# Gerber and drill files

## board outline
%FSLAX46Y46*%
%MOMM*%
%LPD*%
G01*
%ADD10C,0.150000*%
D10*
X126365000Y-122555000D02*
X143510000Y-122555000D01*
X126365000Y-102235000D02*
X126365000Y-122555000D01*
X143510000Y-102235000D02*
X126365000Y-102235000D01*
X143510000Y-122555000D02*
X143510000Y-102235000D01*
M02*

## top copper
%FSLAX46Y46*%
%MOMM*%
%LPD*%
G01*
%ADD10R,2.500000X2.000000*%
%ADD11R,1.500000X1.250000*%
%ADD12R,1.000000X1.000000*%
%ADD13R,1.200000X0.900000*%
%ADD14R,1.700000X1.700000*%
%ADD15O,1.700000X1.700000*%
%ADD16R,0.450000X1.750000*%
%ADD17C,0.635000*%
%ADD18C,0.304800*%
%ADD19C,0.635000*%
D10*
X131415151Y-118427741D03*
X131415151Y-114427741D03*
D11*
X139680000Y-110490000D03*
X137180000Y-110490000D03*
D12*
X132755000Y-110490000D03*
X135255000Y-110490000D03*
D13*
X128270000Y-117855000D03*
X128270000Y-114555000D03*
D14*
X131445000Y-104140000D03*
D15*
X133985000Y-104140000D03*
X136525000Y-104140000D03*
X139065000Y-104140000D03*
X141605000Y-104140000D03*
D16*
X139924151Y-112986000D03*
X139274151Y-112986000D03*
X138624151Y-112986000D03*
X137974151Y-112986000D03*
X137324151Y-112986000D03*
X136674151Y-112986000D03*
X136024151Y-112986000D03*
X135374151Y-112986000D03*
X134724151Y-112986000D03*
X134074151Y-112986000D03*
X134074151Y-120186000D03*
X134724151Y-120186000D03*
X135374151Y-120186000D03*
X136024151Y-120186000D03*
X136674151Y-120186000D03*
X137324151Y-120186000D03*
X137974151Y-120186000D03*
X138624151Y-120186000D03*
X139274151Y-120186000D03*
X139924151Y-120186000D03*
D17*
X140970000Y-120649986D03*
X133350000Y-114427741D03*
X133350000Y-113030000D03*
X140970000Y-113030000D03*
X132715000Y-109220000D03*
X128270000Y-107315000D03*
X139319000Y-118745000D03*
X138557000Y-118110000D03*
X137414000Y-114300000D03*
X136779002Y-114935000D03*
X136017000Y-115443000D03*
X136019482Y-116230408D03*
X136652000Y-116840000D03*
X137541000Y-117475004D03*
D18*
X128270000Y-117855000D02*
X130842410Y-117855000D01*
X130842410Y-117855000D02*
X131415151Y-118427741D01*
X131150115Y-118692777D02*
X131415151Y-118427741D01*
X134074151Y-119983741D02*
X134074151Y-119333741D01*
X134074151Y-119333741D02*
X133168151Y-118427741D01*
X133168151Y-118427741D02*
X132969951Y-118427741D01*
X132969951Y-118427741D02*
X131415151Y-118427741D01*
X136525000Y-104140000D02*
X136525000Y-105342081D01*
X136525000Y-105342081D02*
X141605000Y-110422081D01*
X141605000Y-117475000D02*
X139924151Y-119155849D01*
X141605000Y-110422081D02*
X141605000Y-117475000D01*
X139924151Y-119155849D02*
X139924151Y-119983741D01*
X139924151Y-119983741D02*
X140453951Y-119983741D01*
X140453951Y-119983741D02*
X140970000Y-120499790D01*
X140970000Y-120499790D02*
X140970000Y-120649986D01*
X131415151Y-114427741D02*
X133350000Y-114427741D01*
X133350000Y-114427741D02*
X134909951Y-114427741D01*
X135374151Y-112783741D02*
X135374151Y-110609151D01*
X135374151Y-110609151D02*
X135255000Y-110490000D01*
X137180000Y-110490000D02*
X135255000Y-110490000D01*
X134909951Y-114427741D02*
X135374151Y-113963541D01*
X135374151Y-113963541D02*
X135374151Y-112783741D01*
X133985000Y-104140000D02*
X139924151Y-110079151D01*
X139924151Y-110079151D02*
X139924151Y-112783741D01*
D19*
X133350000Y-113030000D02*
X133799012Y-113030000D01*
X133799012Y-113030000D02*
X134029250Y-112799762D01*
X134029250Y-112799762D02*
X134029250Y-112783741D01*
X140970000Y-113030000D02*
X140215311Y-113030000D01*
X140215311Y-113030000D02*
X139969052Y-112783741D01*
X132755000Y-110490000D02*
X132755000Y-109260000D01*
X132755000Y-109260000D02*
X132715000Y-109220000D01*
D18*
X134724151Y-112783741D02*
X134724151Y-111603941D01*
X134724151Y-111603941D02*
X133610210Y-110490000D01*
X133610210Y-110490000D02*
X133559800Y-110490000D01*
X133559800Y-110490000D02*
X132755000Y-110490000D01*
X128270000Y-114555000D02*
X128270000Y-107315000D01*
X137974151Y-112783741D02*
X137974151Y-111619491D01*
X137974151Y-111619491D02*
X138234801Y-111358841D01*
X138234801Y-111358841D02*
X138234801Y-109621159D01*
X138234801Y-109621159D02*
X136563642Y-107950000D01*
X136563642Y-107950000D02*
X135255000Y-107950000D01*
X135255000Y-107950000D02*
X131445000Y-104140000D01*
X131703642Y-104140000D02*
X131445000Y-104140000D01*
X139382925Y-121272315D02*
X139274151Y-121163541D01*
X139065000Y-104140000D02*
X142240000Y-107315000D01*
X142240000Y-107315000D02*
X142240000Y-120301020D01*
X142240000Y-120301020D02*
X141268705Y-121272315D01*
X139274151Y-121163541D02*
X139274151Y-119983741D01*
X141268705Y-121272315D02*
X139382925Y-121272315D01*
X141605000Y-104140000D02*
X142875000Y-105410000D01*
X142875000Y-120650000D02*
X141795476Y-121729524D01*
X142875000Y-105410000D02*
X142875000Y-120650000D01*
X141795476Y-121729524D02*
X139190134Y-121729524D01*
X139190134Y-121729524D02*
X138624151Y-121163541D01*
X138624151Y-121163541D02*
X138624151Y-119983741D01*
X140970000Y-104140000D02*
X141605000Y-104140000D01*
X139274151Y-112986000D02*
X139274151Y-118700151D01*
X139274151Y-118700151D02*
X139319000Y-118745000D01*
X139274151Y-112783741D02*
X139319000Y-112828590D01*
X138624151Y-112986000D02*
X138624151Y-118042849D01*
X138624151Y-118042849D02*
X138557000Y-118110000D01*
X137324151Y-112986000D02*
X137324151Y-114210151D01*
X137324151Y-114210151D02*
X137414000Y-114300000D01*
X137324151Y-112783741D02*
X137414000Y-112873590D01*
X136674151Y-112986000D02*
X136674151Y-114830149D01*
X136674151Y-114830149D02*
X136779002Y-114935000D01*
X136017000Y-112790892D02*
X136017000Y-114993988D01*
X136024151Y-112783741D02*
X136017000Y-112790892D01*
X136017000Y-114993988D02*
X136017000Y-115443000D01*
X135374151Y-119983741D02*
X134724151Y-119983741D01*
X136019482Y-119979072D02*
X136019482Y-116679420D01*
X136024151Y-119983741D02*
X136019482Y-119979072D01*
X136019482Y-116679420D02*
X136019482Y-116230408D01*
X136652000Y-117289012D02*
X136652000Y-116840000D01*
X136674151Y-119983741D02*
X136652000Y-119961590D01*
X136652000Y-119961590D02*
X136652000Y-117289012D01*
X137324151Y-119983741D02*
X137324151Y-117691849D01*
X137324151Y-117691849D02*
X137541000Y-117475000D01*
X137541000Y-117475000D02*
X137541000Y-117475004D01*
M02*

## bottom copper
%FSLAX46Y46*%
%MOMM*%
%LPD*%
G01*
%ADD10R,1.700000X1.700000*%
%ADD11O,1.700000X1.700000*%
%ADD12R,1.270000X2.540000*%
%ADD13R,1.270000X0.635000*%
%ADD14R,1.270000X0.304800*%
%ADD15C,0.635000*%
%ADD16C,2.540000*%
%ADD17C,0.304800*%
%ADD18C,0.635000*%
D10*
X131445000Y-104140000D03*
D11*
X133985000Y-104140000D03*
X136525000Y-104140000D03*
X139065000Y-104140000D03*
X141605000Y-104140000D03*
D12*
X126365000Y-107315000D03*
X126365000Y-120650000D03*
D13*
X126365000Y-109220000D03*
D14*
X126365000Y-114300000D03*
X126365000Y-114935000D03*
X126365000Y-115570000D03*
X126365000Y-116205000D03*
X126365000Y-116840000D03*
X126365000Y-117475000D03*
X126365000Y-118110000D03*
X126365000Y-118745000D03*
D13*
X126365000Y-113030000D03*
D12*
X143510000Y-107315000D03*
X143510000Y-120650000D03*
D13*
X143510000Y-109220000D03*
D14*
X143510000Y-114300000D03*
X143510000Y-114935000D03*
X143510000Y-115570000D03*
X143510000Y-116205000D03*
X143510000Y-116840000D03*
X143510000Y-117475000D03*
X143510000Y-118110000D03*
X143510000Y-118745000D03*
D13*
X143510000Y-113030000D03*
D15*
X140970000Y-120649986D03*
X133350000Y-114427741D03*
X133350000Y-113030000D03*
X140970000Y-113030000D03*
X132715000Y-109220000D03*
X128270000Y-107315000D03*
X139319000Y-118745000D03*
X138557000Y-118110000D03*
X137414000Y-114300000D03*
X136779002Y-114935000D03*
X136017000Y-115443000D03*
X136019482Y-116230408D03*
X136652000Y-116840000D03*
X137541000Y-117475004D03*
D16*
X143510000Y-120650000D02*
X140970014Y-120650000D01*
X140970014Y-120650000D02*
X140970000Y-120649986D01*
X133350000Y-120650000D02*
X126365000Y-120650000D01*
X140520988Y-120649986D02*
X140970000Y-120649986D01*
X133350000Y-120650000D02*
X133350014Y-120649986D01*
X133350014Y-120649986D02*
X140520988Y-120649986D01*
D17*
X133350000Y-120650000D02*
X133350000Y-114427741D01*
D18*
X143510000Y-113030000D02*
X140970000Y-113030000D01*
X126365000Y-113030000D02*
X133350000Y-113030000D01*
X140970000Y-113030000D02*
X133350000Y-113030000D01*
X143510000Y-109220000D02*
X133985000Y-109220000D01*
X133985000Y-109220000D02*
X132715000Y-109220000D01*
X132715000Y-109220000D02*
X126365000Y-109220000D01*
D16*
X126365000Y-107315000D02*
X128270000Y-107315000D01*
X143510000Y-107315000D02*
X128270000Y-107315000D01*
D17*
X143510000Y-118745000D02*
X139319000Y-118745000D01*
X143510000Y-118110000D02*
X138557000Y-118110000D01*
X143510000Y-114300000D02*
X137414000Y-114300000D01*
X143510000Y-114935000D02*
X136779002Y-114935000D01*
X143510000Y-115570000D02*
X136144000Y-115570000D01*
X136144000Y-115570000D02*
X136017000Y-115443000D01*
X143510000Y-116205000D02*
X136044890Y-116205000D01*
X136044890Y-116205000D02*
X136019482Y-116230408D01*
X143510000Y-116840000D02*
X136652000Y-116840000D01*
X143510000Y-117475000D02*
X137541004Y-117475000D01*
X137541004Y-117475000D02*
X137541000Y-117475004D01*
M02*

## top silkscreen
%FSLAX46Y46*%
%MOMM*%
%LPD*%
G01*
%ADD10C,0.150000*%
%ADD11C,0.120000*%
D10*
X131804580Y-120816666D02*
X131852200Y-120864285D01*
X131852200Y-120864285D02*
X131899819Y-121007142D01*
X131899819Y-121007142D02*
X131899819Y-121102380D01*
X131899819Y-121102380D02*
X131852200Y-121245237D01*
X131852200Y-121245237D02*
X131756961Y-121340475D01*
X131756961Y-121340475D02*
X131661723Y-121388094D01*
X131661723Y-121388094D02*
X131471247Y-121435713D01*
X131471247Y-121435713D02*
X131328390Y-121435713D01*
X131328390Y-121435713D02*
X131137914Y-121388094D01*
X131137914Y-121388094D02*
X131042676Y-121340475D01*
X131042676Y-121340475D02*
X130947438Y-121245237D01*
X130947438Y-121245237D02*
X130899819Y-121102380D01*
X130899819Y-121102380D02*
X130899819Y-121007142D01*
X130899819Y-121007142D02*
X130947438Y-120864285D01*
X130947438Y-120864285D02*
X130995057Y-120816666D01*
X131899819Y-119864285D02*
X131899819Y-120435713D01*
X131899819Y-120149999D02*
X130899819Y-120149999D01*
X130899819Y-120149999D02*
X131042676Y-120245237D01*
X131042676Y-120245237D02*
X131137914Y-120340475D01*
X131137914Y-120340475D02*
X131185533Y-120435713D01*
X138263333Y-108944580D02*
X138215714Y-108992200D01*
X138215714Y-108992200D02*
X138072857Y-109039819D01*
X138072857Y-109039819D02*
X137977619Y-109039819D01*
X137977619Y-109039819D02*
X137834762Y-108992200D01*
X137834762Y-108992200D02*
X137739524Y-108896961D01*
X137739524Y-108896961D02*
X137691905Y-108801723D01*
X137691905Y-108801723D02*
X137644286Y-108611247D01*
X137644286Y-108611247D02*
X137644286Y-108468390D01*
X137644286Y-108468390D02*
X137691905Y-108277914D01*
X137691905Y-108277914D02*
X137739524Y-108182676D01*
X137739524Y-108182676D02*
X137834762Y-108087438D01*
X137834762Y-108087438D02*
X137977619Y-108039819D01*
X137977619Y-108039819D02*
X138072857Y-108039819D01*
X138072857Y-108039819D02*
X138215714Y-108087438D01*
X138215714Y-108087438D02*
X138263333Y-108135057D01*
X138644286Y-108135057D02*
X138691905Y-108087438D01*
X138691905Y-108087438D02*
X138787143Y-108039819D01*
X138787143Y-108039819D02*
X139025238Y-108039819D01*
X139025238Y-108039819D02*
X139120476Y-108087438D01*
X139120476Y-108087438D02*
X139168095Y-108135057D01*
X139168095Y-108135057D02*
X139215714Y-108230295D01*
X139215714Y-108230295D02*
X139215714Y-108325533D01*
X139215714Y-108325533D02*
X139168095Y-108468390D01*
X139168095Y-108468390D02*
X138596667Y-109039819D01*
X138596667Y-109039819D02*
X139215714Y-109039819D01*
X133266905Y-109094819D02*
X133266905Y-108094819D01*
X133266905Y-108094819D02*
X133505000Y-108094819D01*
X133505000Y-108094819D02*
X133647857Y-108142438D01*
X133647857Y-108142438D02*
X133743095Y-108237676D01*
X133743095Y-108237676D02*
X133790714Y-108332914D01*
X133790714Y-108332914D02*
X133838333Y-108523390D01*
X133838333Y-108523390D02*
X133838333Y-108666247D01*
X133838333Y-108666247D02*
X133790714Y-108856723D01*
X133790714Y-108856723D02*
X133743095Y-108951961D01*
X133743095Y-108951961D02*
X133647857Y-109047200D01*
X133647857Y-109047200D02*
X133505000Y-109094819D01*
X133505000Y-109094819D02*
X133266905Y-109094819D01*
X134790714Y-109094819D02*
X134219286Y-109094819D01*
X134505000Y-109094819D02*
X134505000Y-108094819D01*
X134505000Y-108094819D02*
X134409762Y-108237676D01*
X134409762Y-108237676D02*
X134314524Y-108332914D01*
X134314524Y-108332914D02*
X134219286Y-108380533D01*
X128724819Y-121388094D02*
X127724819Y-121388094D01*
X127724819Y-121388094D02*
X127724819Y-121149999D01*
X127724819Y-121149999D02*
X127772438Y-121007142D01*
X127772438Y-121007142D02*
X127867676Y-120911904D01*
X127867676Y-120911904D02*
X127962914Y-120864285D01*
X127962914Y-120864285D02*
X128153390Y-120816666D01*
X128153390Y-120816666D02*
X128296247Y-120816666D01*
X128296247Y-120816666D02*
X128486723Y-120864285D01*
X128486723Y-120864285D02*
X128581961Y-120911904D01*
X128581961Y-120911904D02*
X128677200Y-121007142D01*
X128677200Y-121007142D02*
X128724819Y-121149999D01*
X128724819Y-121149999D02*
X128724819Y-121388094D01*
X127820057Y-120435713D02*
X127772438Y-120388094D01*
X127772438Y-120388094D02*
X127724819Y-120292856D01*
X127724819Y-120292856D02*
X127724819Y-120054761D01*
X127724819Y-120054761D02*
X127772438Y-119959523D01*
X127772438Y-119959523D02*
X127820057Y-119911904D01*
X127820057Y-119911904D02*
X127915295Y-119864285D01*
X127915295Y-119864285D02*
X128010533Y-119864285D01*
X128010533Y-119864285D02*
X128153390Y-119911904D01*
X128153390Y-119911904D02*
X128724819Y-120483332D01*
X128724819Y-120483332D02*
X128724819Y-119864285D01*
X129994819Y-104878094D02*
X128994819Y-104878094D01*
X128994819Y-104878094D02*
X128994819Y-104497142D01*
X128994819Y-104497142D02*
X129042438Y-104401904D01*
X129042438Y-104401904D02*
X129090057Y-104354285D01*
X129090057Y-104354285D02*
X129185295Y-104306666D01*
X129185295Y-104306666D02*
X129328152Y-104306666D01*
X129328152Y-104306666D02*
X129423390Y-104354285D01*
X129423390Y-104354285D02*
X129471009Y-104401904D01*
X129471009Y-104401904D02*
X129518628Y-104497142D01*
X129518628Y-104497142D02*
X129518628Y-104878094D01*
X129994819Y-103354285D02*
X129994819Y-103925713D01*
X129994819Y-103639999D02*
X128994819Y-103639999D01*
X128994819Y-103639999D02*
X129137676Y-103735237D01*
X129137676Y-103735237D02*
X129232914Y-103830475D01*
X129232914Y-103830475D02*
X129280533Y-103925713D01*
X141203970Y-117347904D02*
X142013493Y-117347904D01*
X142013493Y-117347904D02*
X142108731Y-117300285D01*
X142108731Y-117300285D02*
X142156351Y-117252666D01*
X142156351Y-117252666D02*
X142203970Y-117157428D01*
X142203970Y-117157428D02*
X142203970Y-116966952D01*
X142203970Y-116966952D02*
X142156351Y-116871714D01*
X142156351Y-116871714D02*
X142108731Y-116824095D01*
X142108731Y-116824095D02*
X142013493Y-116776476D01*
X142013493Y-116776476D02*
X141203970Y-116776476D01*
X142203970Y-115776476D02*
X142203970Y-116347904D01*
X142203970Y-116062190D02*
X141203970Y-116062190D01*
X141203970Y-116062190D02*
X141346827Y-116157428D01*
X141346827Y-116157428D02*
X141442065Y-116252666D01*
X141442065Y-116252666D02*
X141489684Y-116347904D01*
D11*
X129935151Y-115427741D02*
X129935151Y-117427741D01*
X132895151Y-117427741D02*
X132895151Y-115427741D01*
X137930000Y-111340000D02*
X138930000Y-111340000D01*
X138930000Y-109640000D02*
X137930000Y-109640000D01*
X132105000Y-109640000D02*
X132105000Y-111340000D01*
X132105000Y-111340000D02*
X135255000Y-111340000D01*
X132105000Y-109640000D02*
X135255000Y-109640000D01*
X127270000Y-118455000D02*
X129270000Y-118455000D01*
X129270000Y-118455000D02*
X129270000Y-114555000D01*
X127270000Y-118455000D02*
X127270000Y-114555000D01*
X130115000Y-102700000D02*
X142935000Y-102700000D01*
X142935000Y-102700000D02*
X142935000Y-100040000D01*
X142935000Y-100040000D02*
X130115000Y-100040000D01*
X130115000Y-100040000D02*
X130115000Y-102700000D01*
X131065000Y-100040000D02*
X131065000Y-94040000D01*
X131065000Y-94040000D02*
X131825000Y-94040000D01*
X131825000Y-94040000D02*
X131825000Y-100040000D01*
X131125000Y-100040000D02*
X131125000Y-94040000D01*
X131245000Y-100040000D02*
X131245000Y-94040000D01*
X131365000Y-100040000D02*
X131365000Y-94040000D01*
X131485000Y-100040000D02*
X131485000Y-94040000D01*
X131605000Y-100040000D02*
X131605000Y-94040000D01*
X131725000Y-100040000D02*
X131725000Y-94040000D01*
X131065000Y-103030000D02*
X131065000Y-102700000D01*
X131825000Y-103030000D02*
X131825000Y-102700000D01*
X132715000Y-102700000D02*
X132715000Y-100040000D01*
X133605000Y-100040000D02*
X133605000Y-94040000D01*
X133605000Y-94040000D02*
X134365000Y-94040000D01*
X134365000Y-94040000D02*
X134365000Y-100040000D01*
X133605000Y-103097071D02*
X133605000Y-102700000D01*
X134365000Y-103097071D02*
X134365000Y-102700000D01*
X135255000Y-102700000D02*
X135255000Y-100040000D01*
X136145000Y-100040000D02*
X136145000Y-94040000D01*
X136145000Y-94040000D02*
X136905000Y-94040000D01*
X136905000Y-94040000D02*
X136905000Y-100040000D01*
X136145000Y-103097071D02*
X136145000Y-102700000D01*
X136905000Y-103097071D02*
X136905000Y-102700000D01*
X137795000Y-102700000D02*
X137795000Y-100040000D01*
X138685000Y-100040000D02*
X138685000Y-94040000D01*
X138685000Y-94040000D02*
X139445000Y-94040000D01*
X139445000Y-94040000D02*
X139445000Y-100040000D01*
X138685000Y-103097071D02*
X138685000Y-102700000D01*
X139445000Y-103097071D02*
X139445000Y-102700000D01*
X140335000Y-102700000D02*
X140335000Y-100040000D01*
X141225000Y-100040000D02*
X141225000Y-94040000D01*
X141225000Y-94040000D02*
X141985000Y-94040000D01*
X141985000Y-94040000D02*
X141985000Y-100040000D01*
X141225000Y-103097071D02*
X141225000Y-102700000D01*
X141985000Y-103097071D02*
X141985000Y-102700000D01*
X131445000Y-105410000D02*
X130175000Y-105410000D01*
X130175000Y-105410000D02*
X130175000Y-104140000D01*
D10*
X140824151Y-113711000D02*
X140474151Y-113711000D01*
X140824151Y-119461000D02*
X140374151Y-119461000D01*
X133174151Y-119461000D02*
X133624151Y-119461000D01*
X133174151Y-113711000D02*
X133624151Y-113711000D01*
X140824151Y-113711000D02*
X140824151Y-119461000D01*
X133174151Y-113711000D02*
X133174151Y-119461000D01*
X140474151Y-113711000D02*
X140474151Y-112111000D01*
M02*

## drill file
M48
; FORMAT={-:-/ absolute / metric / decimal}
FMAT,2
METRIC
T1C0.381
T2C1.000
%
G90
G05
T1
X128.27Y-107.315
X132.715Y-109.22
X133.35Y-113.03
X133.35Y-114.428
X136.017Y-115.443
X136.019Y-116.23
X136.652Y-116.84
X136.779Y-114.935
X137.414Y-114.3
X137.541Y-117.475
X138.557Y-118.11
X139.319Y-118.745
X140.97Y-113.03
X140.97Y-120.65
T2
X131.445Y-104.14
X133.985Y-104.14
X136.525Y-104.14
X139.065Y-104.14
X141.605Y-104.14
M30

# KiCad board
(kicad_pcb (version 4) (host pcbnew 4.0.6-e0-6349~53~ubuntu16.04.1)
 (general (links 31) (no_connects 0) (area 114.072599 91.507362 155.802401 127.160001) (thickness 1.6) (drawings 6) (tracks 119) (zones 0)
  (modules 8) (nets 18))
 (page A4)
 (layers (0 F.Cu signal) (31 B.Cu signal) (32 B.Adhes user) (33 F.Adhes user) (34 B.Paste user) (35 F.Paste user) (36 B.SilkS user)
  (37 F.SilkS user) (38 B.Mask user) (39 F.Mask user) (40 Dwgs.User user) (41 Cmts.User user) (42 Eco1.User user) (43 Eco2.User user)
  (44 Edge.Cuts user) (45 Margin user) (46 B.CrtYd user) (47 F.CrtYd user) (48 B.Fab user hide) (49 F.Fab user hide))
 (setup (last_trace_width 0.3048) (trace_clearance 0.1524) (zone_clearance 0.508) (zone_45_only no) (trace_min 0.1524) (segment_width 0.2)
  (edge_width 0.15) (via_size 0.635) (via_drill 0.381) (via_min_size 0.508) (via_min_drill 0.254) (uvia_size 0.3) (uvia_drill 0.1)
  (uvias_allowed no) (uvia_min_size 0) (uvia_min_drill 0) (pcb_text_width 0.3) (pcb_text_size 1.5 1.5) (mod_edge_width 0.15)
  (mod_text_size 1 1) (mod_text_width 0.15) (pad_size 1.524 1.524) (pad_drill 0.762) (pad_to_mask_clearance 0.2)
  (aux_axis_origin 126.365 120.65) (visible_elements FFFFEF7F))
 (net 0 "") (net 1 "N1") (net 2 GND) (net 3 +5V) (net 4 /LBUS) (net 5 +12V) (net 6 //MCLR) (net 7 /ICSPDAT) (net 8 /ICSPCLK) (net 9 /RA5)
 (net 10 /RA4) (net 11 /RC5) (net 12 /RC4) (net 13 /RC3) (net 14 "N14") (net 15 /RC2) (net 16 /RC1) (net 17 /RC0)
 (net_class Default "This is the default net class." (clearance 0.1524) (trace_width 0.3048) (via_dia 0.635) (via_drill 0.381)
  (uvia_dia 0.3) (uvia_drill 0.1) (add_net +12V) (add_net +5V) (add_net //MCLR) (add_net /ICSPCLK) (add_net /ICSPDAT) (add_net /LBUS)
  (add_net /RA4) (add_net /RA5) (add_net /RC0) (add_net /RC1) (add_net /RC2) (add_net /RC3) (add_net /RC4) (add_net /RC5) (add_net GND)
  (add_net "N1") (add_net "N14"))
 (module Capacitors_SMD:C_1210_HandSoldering (layer F.Cu) (at 131.415151 116.427741 90)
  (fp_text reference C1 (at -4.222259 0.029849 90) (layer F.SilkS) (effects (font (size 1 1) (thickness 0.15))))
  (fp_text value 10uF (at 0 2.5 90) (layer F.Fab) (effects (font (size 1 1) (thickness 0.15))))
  (fp_line (start 1 -1.48) (end -1 -1.48) (layer F.SilkS) (width 0.12))
  (fp_line (start -1 1.48) (end 1 1.48) (layer F.SilkS) (width 0.12))
  (pad 1 smd rect (at -2 0 90) (size 2 2.5) (layers F.Cu F.Paste F.Mask) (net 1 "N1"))
  (pad 2 smd rect (at 2 0 90) (size 2 2.5) (layers F.Cu F.Paste F.Mask) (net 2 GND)))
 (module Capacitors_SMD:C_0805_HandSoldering (layer F.Cu) (at 138.43 110.49 180)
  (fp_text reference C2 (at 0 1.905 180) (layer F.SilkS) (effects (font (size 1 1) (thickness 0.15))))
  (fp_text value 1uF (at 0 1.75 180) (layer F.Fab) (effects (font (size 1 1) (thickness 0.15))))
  (fp_line (start 0.5 -0.85) (end -0.5 -0.85) (layer F.SilkS) (width 0.12))
  (fp_line (start -0.5 0.85) (end 0.5 0.85) (layer F.SilkS) (width 0.12))
  (pad 1 smd rect (at -1.25 0 180) (size 1.5 1.25) (layers F.Cu F.Paste F.Mask) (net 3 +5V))
  (pad 2 smd rect (at 1.25 0 180) (size 1.5 1.25) (layers F.Cu F.Paste F.Mask) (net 2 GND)))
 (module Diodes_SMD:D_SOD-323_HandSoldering (layer F.Cu) (at 134.005 110.49)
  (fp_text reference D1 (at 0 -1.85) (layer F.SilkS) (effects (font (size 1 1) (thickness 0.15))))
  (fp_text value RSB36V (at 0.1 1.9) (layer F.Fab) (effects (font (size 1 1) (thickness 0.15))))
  (fp_line (start -1.9 -0.85) (end -1.9 0.85) (layer F.SilkS) (width 0.12))
  (fp_line (start -1.9 0.85) (end 1.25 0.85) (layer F.SilkS) (width 0.12))
  (fp_line (start -1.9 -0.85) (end 1.25 -0.85) (layer F.SilkS) (width 0.12))
  (pad 1 smd rect (at -1.25 0) (size 1 1) (layers F.Cu F.Paste F.Mask) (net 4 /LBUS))
  (pad 2 smd rect (at 1.25 0) (size 1 1) (layers F.Cu F.Paste F.Mask) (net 2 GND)))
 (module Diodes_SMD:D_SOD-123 (layer F.Cu) (at 128.27 116.205 90)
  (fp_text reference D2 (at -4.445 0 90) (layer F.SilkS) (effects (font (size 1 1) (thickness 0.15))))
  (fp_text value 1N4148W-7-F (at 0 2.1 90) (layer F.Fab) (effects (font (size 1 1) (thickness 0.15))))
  (fp_line (start -2.25 -1) (end -2.25 1) (layer F.SilkS) (width 0.12))
  (fp_line (start -2.25 1) (end 1.65 1) (layer F.SilkS) (width 0.12))
  (fp_line (start -2.25 -1) (end 1.65 -1) (layer F.SilkS) (width 0.12))
  (pad 1 smd rect (at -1.65 0 90) (size 0.9 1.2) (layers F.Cu F.Paste F.Mask) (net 1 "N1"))
  (pad 2 smd rect (at 1.65 0 90) (size 0.9 1.2) (layers F.Cu F.Paste F.Mask) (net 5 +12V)))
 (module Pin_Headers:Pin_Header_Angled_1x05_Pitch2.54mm (layer F.Cu) (at 131.445 104.14 90)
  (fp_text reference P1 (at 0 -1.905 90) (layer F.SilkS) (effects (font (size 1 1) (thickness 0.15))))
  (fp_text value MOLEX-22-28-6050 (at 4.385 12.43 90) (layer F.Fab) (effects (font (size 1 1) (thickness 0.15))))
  (fp_line (start 1.44 -1.33) (end 1.44 11.49) (layer F.SilkS) (width 0.12))
  (fp_line (start 1.44 11.49) (end 4.1 11.49) (layer F.SilkS) (width 0.12))
  (fp_line (start 4.1 11.49) (end 4.1 -1.33) (layer F.SilkS) (width 0.12))
  (fp_line (start 4.1 -1.33) (end 1.44 -1.33) (layer F.SilkS) (width 0.12))
  (fp_line (start 4.1 -0.38) (end 10.1 -0.38) (layer F.SilkS) (width 0.12))
  (fp_line (start 10.1 -0.38) (end 10.1 0.38) (layer F.SilkS) (width 0.12))
  (fp_line (start 10.1 0.38) (end 4.1 0.38) (layer F.SilkS) (width 0.12))
  (fp_line (start 4.1 -0.32) (end 10.1 -0.32) (layer F.SilkS) (width 0.12))
  (fp_line (start 4.1 -0.2) (end 10.1 -0.2) (layer F.SilkS) (width 0.12))
  (fp_line (start 4.1 -0.08) (end 10.1 -0.08) (layer F.SilkS) (width 0.12))
  (fp_line (start 4.1 0.04) (end 10.1 0.04) (layer F.SilkS) (width 0.12))
  (fp_line (start 4.1 0.16) (end 10.1 0.16) (layer F.SilkS) (width 0.12))
  (fp_line (start 4.1 0.28) (end 10.1 0.28) (layer F.SilkS) (width 0.12))
  (fp_line (start 1.11 -0.38) (end 1.44 -0.38) (layer F.SilkS) (width 0.12))
  (fp_line (start 1.11 0.38) (end 1.44 0.38) (layer F.SilkS) (width 0.12))
  (fp_line (start 1.44 1.27) (end 4.1 1.27) (layer F.SilkS) (width 0.12))
  (fp_line (start 4.1 2.16) (end 10.1 2.16) (layer F.SilkS) (width 0.12))
  (fp_line (start 10.1 2.16) (end 10.1 2.92) (layer F.SilkS) (width 0.12))
  (fp_line (start 10.1 2.92) (end 4.1 2.92) (layer F.SilkS) (width 0.12))
  (fp_line (start 1.042929 2.16) (end 1.44 2.16) (layer F.SilkS) (width 0.12))
  (fp_line (start 1.042929 2.92) (end 1.44 2.92) (layer F.SilkS) (width 0.12))
  (fp_line (start 1.44 3.81) (end 4.1 3.81) (layer F.SilkS) (width 0.12))
  (fp_line (start 4.1 4.7) (end 10.1 4.7) (layer F.SilkS) (width 0.12))
  (fp_line (start 10.1 4.7) (end 10.1 5.46) (layer F.SilkS) (width 0.12))
  (fp_line (start 10.1 5.46) (end 4.1 5.46) (layer F.SilkS) (width 0.12))
  (fp_line (start 1.042929 4.7) (end 1.44 4.7) (layer F.SilkS) (width 0.12))
  (fp_line (start 1.042929 5.46) (end 1.44 5.46) (layer F.SilkS) (width 0.12))
  (fp_line (start 1.44 6.35) (end 4.1 6.35) (layer F.SilkS) (width 0.12))
  (fp_line (start 4.1 7.24) (end 10.1 7.24) (layer F.SilkS) (width 0.12))
  (fp_line (start 10.1 7.24) (end 10.1 8) (layer F.SilkS) (width 0.12))
  (fp_line (start 10.1 8) (end 4.1 8) (layer F.SilkS) (width 0.12))
  (fp_line (start 1.042929 7.24) (end 1.44 7.24) (layer F.SilkS) (width 0.12))
  (fp_line (start 1.042929 8) (end 1.44 8) (layer F.SilkS) (width 0.12))
  (fp_line (start 1.44 8.89) (end 4.1 8.89) (layer F.SilkS) (width 0.12))
  (fp_line (start 4.1 9.78) (end 10.1 9.78) (layer F.SilkS) (width 0.12))
  (fp_line (start 10.1 9.78) (end 10.1 10.54) (layer F.SilkS) (width 0.12))
  (fp_line (start 10.1 10.54) (end 4.1 10.54) (layer F.SilkS) (width 0.12))
  (fp_line (start 1.042929 9.78) (end 1.44 9.78) (layer F.SilkS) (width 0.12))
  (fp_line (start 1.042929 10.54) (end 1.44 10.54) (layer F.SilkS) (width 0.12))
  (fp_line (start -1.27 0) (end -1.27 -1.27) (layer F.SilkS) (width 0.12))
  (fp_line (start -1.27 -1.27) (end 0 -1.27) (layer F.SilkS) (width 0.12))
  (pad 1 thru_hole rect (at 0 0 90) (size 1.7 1.7) (drill 1) (layers *.Cu *.Mask) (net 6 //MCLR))
  (pad 2 thru_hole oval (at 0 2.54 90) (size 1.7 1.7) (drill 1) (layers *.Cu *.Mask) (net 3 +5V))
  (pad 3 thru_hole oval (at 0 5.08 90) (size 1.7 1.7) (drill 1) (layers *.Cu *.Mask) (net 2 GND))
  (pad 4 thru_hole oval (at 0 7.62 90) (size 1.7 1.7) (drill 1) (layers *.Cu *.Mask) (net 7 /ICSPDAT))
  (pad 5 thru_hole oval (at 0 10.16 90) (size 1.7 1.7) (drill 1) (layers *.Cu *.Mask) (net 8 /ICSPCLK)))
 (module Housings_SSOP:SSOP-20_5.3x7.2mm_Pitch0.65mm (layer F.Cu) (at 136.999151 116.586 270)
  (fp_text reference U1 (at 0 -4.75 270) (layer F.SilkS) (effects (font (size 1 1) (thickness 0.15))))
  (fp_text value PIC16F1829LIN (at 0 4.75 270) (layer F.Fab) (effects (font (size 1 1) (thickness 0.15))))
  (fp_line (start -2.875 -3.825) (end -2.875 -3.475) (layer F.SilkS) (width 0.15))
  (fp_line (start 2.875 -3.825) (end 2.875 -3.375) (layer F.SilkS) (width 0.15))
  (fp_line (start 2.875 3.825) (end 2.875 3.375) (layer F.SilkS) (width 0.15))
  (fp_line (start -2.875 3.825) (end -2.875 3.375) (layer F.SilkS) (width 0.15))
  (fp_line (start -2.875 -3.825) (end 2.875 -3.825) (layer F.SilkS) (width 0.15))
  (fp_line (start -2.875 3.825) (end 2.875 3.825) (layer F.SilkS) (width 0.15))
  (fp_line (start -2.875 -3.475) (end -4.475 -3.475) (layer F.SilkS) (width 0.15))
  (pad 1 smd rect (at -3.6 -2.925 270) (size 1.75 0.45) (layers F.Cu F.Paste F.Mask) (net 3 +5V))
  (pad 2 smd rect (at -3.6 -2.275 270) (size 1.75 0.45) (layers F.Cu F.Paste F.Mask) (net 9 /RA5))
  (pad 3 smd rect (at -3.6 -1.625 270) (size 1.75 0.45) (layers F.Cu F.Paste F.Mask) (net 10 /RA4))
  (pad 4 smd rect (at -3.6 -0.975 270) (size 1.75 0.45) (layers F.Cu F.Paste F.Mask) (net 6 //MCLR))
  (pad 5 smd rect (at -3.6 -0.325 270) (size 1.75 0.45) (layers F.Cu F.Paste F.Mask) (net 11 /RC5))
  (pad 6 smd rect (at -3.6 0.325 270) (size 1.75 0.45) (layers F.Cu F.Paste F.Mask) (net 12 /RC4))
  (pad 7 smd rect (at -3.6 0.975 270) (size 1.75 0.45) (layers F.Cu F.Paste F.Mask) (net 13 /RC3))
  (pad 8 smd rect (at -3.6 1.625 270) (size 1.75 0.45) (layers F.Cu F.Paste F.Mask) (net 2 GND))
  (pad 9 smd rect (at -3.6 2.275 270) (size 1.75 0.45) (layers F.Cu F.Paste F.Mask) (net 4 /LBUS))
  (pad 10 smd rect (at -3.6 2.925 270) (size 1.75 0.45) (layers F.Cu F.Paste F.Mask) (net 3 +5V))
  (pad 11 smd rect (at 3.6 2.925 270) (size 1.75 0.45) (layers F.Cu F.Paste F.Mask) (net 1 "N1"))
  (pad 12 smd rect (at 3.6 2.275 270) (size 1.75 0.45) (layers F.Cu F.Paste F.Mask) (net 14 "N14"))
  (pad 13 smd rect (at 3.6 1.625 270) (size 1.75 0.45) (layers F.Cu F.Paste F.Mask) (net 14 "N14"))
  (pad 14 smd rect (at 3.6 0.975 270) (size 1.75 0.45) (layers F.Cu F.Paste F.Mask) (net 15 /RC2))
  (pad 15 smd rect (at 3.6 0.325 270) (size 1.75 0.45) (layers F.Cu F.Paste F.Mask) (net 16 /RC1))
  (pad 16 smd rect (at 3.6 -0.325 270) (size 1.75 0.45) (layers F.Cu F.Paste F.Mask) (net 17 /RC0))
  (pad 17 smd rect (at 3.6 -0.975 270) (size 1.75 0.45) (layers F.Cu F.Paste F.Mask))
  (pad 18 smd rect (at 3.6 -1.625 270) (size 1.75 0.45) (layers F.Cu F.Paste F.Mask) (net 8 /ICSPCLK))
  (pad 19 smd rect (at 3.6 -2.275 270) (size 1.75 0.45) (layers F.Cu F.Paste F.Mask) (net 7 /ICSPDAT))
  (pad 20 smd rect (at 3.6 -2.925 270) (size 1.75 0.45) (layers F.Cu F.Paste F.Mask) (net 2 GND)))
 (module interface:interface (layer F.Cu) (at 126.365 102.87)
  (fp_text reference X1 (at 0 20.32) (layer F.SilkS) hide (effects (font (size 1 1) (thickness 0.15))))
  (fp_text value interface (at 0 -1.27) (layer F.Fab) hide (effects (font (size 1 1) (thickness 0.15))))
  (pad 1 smd rect (at 0 4.445) (size 1.27 2.54) (layers B.Cu) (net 5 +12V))
  (pad 2 smd rect (at 0 17.78) (size 1.27 2.54) (layers B.Cu) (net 2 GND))
  (pad 3 smd rect (at 0 6.35) (size 1.27 0.635) (layers B.Cu) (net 4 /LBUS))
  (pad 5 smd rect (at 0 11.43) (size 1.27 0.3048) (layers B.Cu))
  (pad 6 smd rect (at 0 12.065) (size 1.27 0.3048) (layers B.Cu))
  (pad 7 smd rect (at 0 12.7) (size 1.27 0.3048) (layers B.Cu))
  (pad 8 smd rect (at 0 13.335) (size 1.27 0.3048) (layers B.Cu))
  (pad 9 smd rect (at 0 13.97) (size 1.27 0.3048) (layers B.Cu))
  (pad 10 smd rect (at 0 14.605) (size 1.27 0.3048) (layers B.Cu))
  (pad 11 smd rect (at 0 15.24) (size 1.27 0.3048) (layers B.Cu))
  (pad 12 smd rect (at 0 15.875) (size 1.27 0.3048) (layers B.Cu))
  (pad 4 smd rect (at 0 10.16) (size 1.27 0.635) (layers B.Cu) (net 3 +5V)))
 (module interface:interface (layer F.Cu) (at 143.51 102.87)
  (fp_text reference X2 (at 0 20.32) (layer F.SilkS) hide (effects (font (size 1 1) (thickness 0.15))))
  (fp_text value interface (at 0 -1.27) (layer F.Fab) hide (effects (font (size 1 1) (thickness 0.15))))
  (pad 1 smd rect (at 0 4.445) (size 1.27 2.54) (layers B.Cu) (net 5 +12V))
  (pad 2 smd rect (at 0 17.78) (size 1.27 2.54) (layers B.Cu) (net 2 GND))
  (pad 3 smd rect (at 0 6.35) (size 1.27 0.635) (layers B.Cu) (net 4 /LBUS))
  (pad 5 smd rect (at 0 11.43) (size 1.27 0.3048) (layers B.Cu) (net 11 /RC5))
  (pad 6 smd rect (at 0 12.065) (size 1.27 0.3048) (layers B.Cu) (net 12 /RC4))
  (pad 7 smd rect (at 0 12.7) (size 1.27 0.3048) (layers B.Cu) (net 13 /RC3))
  (pad 8 smd rect (at 0 13.335) (size 1.27 0.3048) (layers B.Cu) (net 15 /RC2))
  (pad 9 smd rect (at 0 13.97) (size 1.27 0.3048) (layers B.Cu) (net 16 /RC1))
  (pad 10 smd rect (at 0 14.605) (size 1.27 0.3048) (layers B.Cu) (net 17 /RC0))
  (pad 11 smd rect (at 0 15.24) (size 1.27 0.3048) (layers B.Cu) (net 10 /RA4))
  (pad 12 smd rect (at 0 15.875) (size 1.27 0.3048) (layers B.Cu) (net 9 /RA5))
  (pad 4 smd rect (at 0 10.16) (size 1.27 0.635) (layers B.Cu) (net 3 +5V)))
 (gr_line (start 126.365 122.555) (end 143.51 122.555) (layer Edge.Cuts) (width 0.15))
 (gr_line (start 126.365 102.235) (end 126.365 122.555) (layer Edge.Cuts) (width 0.15))
 (gr_line (start 143.51 102.235) (end 126.365 102.235) (layer Edge.Cuts) (width 0.15))
 (gr_line (start 143.51 122.555) (end 143.51 102.235) (layer Edge.Cuts) (width 0.15))
 (segment (start 128.27 117.855) (end 130.84241 117.855) (width 0.3048) (layer F.Cu) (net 1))
 (segment (start 130.84241 117.855) (end 131.415151 118.427741) (width 0.3048) (layer F.Cu) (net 1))
 (segment (start 131.150115 118.692777) (end 131.415151 118.427741) (width 0.3048) (layer F.Cu) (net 1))
 (segment (start 134.074151 119.983741) (end 134.074151 119.333741) (width 0.3048) (layer F.Cu) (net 1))
 (segment (start 134.074151 119.333741) (end 133.168151 118.427741) (width 0.3048) (layer F.Cu) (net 1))
 (segment (start 133.168151 118.427741) (end 132.969951 118.427741) (width 0.3048) (layer F.Cu) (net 1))
 (segment (start 132.969951 118.427741) (end 131.415151 118.427741) (width 0.3048) (layer F.Cu) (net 1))
 (segment (start 143.51 120.65) (end 140.970014 120.65) (width 2.54) (layer B.Cu) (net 2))
 (segment (start 140.970014 120.65) (end 140.97 120.649986) (width 2.54) (layer B.Cu) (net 2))
 (segment (start 133.35 120.65) (end 126.365 120.65) (width 2.54) (layer B.Cu) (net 2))
 (segment (start 136.525 104.14) (end 136.525 105.342081) (width 0.3048) (layer F.Cu) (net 2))
 (segment (start 136.525 105.342081) (end 141.605 110.422081) (width 0.3048) (layer F.Cu) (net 2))
 (segment (start 141.605 117.475) (end 139.924151 119.155849) (width 0.3048) (layer F.Cu) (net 2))
 (segment (start 141.605 110.422081) (end 141.605 117.475) (width 0.3048) (layer F.Cu) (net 2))
 (segment (start 139.924151 119.155849) (end 139.924151 119.983741) (width 0.3048) (layer F.Cu) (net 2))
 (segment (start 139.924151 119.983741) (end 140.453951 119.983741) (width 0.3048) (layer F.Cu) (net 2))
 (segment (start 140.520988 120.649986) (end 140.97 120.649986) (width 2.54) (layer B.Cu) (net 2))
 (segment (start 133.35 120.65) (end 133.350014 120.649986) (width 2.54) (layer B.Cu) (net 2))
 (segment (start 140.453951 119.983741) (end 140.97 120.49979) (width 0.3048) (layer F.Cu) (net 2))
 (via (at 140.97 120.649986) (size 0.635) (drill 0.381) (layers F.Cu B.Cu) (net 2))
 (segment (start 140.97 120.49979) (end 140.97 120.649986) (width 0.3048) (layer F.Cu) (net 2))
 (segment (start 133.350014 120.649986) (end 140.520988 120.649986) (width 2.54) (layer B.Cu) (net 2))
 (segment (start 133.35 120.65) (end 133.35 114.427741) (width 0.3048) (layer B.Cu) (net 2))
 (segment (start 131.415151 114.427741) (end 133.35 114.427741) (width 0.3048) (layer F.Cu) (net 2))
 (segment (start 133.35 114.427741) (end 134.909951 114.427741) (width 0.3048) (layer F.Cu) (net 2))
 (via (at 133.35 114.427741) (size 0.635) (drill 0.381) (layers F.Cu B.Cu) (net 2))
 (segment (start 135.374151 112.783741) (end 135.374151 110.609151) (width 0.3048) (layer F.Cu) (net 2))
 (segment (start 135.374151 110.609151) (end 135.255 110.49) (width 0.3048) (layer F.Cu) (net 2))
 (segment (start 137.18 110.49) (end 135.255 110.49) (width 0.3048) (layer F.Cu) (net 2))
 (segment (start 134.909951 114.427741) (end 135.374151 113.963541) (width 0.3048) (layer F.Cu) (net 2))
 (segment (start 135.374151 113.963541) (end 135.374151 112.783741) (width 0.3048) (layer F.Cu) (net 2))
 (segment (start 143.51 113.03) (end 140.97 113.03) (width 0.635) (layer B.Cu) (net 3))
 (segment (start 126.365 113.03) (end 133.35 113.03) (width 0.635) (layer B.Cu) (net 3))
 (segment (start 133.985 104.14) (end 139.924151 110.079151) (width 0.3048) (layer F.Cu) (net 3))
 (segment (start 139.924151 110.079151) (end 139.924151 112.783741) (width 0.3048) (layer F.Cu) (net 3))
 (segment (start 133.35 113.03) (end 133.799012 113.03) (width 0.635) (layer F.Cu) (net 3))
 (segment (start 133.799012 113.03) (end 134.02925 112.799762) (width 0.635) (layer F.Cu) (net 3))
 (segment (start 134.02925 112.799762) (end 134.02925 112.783741) (width 0.635) (layer F.Cu) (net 3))
 (segment (start 140.97 113.03) (end 133.35 113.03) (width 0.635) (layer B.Cu) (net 3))
 (via (at 133.35 113.03) (size 0.635) (drill 0.381) (layers F.Cu B.Cu) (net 3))
 (segment (start 140.97 113.03) (end 140.215311 113.03) (width 0.635) (layer F.Cu) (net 3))
 (segment (start 140.215311 113.03) (end 139.969052 112.783741) (width 0.635) (layer F.Cu) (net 3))
 (via (at 140.97 113.03) (size 0.635) (drill 0.381) (layers F.Cu B.Cu) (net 3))
 (segment (start 143.51 109.22) (end 133.985 109.22) (width 0.635) (layer B.Cu) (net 4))
 (segment (start 133.985 109.22) (end 132.715 109.22) (width 0.635) (layer B.Cu) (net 4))
 (segment (start 132.715 109.22) (end 126.365 109.22) (width 0.635) (layer B.Cu) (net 4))
 (segment (start 132.755 110.49) (end 132.755 109.26) (width 0.635) (layer F.Cu) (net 4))
 (segment (start 132.755 109.26) (end 132.715 109.22) (width 0.635) (layer F.Cu) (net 4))
 (via (at 132.715 109.22) (size 0.635) (drill 0.381) (layers F.Cu B.Cu) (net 4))
 (segment (start 134.724151 112.783741) (end 134.724151 111.603941) (width 0.3048) (layer F.Cu) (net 4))
 (segment (start 134.724151 111.603941) (end 133.61021 110.49) (width 0.3048) (layer F.Cu) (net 4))
 (segment (start 133.61021 110.49) (end 133.5598 110.49) (width 0.3048) (layer F.Cu) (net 4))
 (segment (start 133.5598 110.49) (end 132.755 110.49) (width 0.3048) (layer F.Cu) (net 4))
 (segment (start 126.365 107.315) (end 128.27 107.315) (width 2.54) (layer B.Cu) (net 5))
 (segment (start 143.51 107.315) (end 128.27 107.315) (width 2.54) (layer B.Cu) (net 5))
 (segment (start 128.27 114.555) (end 128.27 107.315) (width 0.3048) (layer F.Cu) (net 5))
 (via (at 128.27 107.315) (size 0.635) (drill 0.381) (layers F.Cu B.Cu) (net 5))
 (segment (start 137.974151 112.783741) (end 137.974151 111.619491) (width 0.3048) (layer F.Cu) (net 6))
 (segment (start 137.974151 111.619491) (end 138.234801 111.358841) (width 0.3048) (layer F.Cu) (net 6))
 (segment (start 138.234801 111.358841) (end 138.234801 109.621159) (width 0.3048) (layer F.Cu) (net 6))
 (segment (start 138.234801 109.621159) (end 136.563642 107.95) (width 0.3048) (layer F.Cu) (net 6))
 (segment (start 136.563642 107.95) (end 135.255 107.95) (width 0.3048) (layer F.Cu) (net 6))
 (segment (start 135.255 107.95) (end 131.445 104.14) (width 0.3048) (layer F.Cu) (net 6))
 (segment (start 131.703642 104.14) (end 131.445 104.14) (width 0.3048) (layer F.Cu) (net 6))
 (segment (start 139.382925 121.272315) (end 139.274151 121.163541) (width 0.3048) (layer F.Cu) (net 7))
 (segment (start 139.065 104.14) (end 142.24 107.315) (width 0.3048) (layer F.Cu) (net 7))
 (segment (start 142.24 107.315) (end 142.24 120.30102) (width 0.3048) (layer F.Cu) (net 7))
 (segment (start 142.24 120.30102) (end 141.268705 121.272315) (width 0.3048) (layer F.Cu) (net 7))
 (segment (start 139.274151 121.163541) (end 139.274151 119.983741) (width 0.3048) (layer F.Cu) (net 7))
 (segment (start 141.268705 121.272315) (end 139.382925 121.272315) (width 0.3048) (layer F.Cu) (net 7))
 (segment (start 141.605 104.14) (end 142.875 105.41) (width 0.3048) (layer F.Cu) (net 8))
 (segment (start 142.875 120.65) (end 141.795476 121.729524) (width 0.3048) (layer F.Cu) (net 8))
 (segment (start 142.875 105.41) (end 142.875 120.65) (width 0.3048) (layer F.Cu) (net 8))
 (segment (start 141.795476 121.729524) (end 139.190134 121.729524) (width 0.3048) (layer F.Cu) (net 8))
 (segment (start 139.190134 121.729524) (end 138.624151 121.163541) (width 0.3048) (layer F.Cu) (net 8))
 (segment (start 138.624151 121.163541) (end 138.624151 119.983741) (width 0.3048) (layer F.Cu) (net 8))
 (segment (start 140.97 104.14) (end 141.605 104.14) (width 0.3048) (layer F.Cu) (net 8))
 (segment (start 143.51 118.745) (end 139.319 118.745) (width 0.3048) (layer B.Cu) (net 9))
 (segment (start 139.274151 112.986) (end 139.274151 118.700151) (width 0.3048) (layer F.Cu) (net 9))
 (segment (start 139.274151 118.700151) (end 139.319 118.745) (width 0.3048) (layer F.Cu) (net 9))
 (via (at 139.319 118.745) (size 0.635) (drill 0.381) (layers F.Cu B.Cu) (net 9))
 (segment (start 139.274151 112.783741) (end 139.319 112.82859) (width 0.3048) (layer F.Cu) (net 9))
 (segment (start 143.51 118.11) (end 138.557 118.11) (width 0.3048) (layer B.Cu) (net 10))
 (segment (start 138.624151 112.986) (end 138.624151 118.042849) (width 0.3048) (layer F.Cu) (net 10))
 (segment (start 138.624151 118.042849) (end 138.557 118.11) (width 0.3048) (layer F.Cu) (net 10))
 (via (at 138.557 118.11) (size 0.635) (drill 0.381) (layers F.Cu B.Cu) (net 10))
 (segment (start 143.51 114.3) (end 137.414 114.3) (width 0.3048) (layer B.Cu) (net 11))
 (segment (start 137.324151 112.986) (end 137.324151 114.210151) (width 0.3048) (layer F.Cu) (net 11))
 (segment (start 137.324151 114.210151) (end 137.414 114.3) (width 0.3048) (layer F.Cu) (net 11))
 (segment (start 137.324151 112.783741) (end 137.414 112.87359) (width 0.3048) (layer F.Cu) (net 11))
 (via (at 137.414 114.3) (size 0.635) (drill 0.381) (layers F.Cu B.Cu) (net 11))
 (segment (start 143.51 114.935) (end 136.779002 114.935) (width 0.3048) (layer B.Cu) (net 12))
 (segment (start 136.674151 112.986) (end 136.674151 114.830149) (width 0.3048) (layer F.Cu) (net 12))
 (segment (start 136.674151 114.830149) (end 136.779002 114.935) (width 0.3048) (layer F.Cu) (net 12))
 (via (at 136.779002 114.935) (size 0.635) (drill 0.381) (layers F.Cu B.Cu) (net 12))
 (segment (start 143.51 115.57) (end 136.144 115.57) (width 0.3048) (layer B.Cu) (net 13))
 (segment (start 136.144 115.57) (end 136.017 115.443) (width 0.3048) (layer B.Cu) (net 13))
 (segment (start 136.017 112.790892) (end 136.017 114.993988) (width 0.3048) (layer F.Cu) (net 13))
 (segment (start 136.024151 112.783741) (end 136.017 112.790892) (width 0.3048) (layer F.Cu) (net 13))
 (via (at 136.017 115.443) (size 0.635) (drill 0.381) (layers F.Cu B.Cu) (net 13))
 (segment (start 136.017 114.993988) (end 136.017 115.443) (width 0.3048) (layer F.Cu) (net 13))
 (segment (start 135.374151 119.983741) (end 134.724151 119.983741) (width 0.3048) (layer F.Cu) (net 14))
 (segment (start 143.51 116.205) (end 136.04489 116.205) (width 0.3048) (layer B.Cu) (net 15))
 (segment (start 136.04489 116.205) (end 136.019482 116.230408) (width 0.3048) (layer B.Cu) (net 15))
 (segment (start 136.019482 119.979072) (end 136.019482 116.67942) (width 0.3048) (layer F.Cu) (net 15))
 (segment (start 136.024151 119.983741) (end 136.019482 119.979072) (width 0.3048) (layer F.Cu) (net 15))
 (segment (start 136.019482 116.67942) (end 136.019482 116.230408) (width 0.3048) (layer F.Cu) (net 15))
 (via (at 136.019482 116.230408) (size 0.635) (drill 0.381) (layers F.Cu B.Cu) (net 15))
 (segment (start 143.51 116.84) (end 136.652 116.84) (width 0.3048) (layer B.Cu) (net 16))
 (segment (start 136.652 117.289012) (end 136.652 116.84) (width 0.3048) (layer F.Cu) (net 16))
 (segment (start 136.674151 119.983741) (end 136.652 119.96159) (width 0.3048) (layer F.Cu) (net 16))
 (segment (start 136.652 119.96159) (end 136.652 117.289012) (width 0.3048) (layer F.Cu) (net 16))
 (via (at 136.652 116.84) (size 0.635) (drill 0.381) (layers F.Cu B.Cu) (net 16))
 (segment (start 143.51 117.475) (end 137.541004 117.475) (width 0.3048) (layer B.Cu) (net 17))
 (segment (start 137.541004 117.475) (end 137.541 117.475004) (width 0.3048) (layer B.Cu) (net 17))
 (segment (start 137.324151 119.983741) (end 137.324151 117.691849) (width 0.3048) (layer F.Cu) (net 17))
 (segment (start 137.324151 117.691849) (end 137.541 117.475) (width 0.3048) (layer F.Cu) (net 17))
 (segment (start 137.541 117.475) (end 137.541 117.475004) (width 0.3048) (layer F.Cu) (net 17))
 (via (at 137.541 117.475004) (size 0.635) (drill 0.381) (layers F.Cu B.Cu) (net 17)))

